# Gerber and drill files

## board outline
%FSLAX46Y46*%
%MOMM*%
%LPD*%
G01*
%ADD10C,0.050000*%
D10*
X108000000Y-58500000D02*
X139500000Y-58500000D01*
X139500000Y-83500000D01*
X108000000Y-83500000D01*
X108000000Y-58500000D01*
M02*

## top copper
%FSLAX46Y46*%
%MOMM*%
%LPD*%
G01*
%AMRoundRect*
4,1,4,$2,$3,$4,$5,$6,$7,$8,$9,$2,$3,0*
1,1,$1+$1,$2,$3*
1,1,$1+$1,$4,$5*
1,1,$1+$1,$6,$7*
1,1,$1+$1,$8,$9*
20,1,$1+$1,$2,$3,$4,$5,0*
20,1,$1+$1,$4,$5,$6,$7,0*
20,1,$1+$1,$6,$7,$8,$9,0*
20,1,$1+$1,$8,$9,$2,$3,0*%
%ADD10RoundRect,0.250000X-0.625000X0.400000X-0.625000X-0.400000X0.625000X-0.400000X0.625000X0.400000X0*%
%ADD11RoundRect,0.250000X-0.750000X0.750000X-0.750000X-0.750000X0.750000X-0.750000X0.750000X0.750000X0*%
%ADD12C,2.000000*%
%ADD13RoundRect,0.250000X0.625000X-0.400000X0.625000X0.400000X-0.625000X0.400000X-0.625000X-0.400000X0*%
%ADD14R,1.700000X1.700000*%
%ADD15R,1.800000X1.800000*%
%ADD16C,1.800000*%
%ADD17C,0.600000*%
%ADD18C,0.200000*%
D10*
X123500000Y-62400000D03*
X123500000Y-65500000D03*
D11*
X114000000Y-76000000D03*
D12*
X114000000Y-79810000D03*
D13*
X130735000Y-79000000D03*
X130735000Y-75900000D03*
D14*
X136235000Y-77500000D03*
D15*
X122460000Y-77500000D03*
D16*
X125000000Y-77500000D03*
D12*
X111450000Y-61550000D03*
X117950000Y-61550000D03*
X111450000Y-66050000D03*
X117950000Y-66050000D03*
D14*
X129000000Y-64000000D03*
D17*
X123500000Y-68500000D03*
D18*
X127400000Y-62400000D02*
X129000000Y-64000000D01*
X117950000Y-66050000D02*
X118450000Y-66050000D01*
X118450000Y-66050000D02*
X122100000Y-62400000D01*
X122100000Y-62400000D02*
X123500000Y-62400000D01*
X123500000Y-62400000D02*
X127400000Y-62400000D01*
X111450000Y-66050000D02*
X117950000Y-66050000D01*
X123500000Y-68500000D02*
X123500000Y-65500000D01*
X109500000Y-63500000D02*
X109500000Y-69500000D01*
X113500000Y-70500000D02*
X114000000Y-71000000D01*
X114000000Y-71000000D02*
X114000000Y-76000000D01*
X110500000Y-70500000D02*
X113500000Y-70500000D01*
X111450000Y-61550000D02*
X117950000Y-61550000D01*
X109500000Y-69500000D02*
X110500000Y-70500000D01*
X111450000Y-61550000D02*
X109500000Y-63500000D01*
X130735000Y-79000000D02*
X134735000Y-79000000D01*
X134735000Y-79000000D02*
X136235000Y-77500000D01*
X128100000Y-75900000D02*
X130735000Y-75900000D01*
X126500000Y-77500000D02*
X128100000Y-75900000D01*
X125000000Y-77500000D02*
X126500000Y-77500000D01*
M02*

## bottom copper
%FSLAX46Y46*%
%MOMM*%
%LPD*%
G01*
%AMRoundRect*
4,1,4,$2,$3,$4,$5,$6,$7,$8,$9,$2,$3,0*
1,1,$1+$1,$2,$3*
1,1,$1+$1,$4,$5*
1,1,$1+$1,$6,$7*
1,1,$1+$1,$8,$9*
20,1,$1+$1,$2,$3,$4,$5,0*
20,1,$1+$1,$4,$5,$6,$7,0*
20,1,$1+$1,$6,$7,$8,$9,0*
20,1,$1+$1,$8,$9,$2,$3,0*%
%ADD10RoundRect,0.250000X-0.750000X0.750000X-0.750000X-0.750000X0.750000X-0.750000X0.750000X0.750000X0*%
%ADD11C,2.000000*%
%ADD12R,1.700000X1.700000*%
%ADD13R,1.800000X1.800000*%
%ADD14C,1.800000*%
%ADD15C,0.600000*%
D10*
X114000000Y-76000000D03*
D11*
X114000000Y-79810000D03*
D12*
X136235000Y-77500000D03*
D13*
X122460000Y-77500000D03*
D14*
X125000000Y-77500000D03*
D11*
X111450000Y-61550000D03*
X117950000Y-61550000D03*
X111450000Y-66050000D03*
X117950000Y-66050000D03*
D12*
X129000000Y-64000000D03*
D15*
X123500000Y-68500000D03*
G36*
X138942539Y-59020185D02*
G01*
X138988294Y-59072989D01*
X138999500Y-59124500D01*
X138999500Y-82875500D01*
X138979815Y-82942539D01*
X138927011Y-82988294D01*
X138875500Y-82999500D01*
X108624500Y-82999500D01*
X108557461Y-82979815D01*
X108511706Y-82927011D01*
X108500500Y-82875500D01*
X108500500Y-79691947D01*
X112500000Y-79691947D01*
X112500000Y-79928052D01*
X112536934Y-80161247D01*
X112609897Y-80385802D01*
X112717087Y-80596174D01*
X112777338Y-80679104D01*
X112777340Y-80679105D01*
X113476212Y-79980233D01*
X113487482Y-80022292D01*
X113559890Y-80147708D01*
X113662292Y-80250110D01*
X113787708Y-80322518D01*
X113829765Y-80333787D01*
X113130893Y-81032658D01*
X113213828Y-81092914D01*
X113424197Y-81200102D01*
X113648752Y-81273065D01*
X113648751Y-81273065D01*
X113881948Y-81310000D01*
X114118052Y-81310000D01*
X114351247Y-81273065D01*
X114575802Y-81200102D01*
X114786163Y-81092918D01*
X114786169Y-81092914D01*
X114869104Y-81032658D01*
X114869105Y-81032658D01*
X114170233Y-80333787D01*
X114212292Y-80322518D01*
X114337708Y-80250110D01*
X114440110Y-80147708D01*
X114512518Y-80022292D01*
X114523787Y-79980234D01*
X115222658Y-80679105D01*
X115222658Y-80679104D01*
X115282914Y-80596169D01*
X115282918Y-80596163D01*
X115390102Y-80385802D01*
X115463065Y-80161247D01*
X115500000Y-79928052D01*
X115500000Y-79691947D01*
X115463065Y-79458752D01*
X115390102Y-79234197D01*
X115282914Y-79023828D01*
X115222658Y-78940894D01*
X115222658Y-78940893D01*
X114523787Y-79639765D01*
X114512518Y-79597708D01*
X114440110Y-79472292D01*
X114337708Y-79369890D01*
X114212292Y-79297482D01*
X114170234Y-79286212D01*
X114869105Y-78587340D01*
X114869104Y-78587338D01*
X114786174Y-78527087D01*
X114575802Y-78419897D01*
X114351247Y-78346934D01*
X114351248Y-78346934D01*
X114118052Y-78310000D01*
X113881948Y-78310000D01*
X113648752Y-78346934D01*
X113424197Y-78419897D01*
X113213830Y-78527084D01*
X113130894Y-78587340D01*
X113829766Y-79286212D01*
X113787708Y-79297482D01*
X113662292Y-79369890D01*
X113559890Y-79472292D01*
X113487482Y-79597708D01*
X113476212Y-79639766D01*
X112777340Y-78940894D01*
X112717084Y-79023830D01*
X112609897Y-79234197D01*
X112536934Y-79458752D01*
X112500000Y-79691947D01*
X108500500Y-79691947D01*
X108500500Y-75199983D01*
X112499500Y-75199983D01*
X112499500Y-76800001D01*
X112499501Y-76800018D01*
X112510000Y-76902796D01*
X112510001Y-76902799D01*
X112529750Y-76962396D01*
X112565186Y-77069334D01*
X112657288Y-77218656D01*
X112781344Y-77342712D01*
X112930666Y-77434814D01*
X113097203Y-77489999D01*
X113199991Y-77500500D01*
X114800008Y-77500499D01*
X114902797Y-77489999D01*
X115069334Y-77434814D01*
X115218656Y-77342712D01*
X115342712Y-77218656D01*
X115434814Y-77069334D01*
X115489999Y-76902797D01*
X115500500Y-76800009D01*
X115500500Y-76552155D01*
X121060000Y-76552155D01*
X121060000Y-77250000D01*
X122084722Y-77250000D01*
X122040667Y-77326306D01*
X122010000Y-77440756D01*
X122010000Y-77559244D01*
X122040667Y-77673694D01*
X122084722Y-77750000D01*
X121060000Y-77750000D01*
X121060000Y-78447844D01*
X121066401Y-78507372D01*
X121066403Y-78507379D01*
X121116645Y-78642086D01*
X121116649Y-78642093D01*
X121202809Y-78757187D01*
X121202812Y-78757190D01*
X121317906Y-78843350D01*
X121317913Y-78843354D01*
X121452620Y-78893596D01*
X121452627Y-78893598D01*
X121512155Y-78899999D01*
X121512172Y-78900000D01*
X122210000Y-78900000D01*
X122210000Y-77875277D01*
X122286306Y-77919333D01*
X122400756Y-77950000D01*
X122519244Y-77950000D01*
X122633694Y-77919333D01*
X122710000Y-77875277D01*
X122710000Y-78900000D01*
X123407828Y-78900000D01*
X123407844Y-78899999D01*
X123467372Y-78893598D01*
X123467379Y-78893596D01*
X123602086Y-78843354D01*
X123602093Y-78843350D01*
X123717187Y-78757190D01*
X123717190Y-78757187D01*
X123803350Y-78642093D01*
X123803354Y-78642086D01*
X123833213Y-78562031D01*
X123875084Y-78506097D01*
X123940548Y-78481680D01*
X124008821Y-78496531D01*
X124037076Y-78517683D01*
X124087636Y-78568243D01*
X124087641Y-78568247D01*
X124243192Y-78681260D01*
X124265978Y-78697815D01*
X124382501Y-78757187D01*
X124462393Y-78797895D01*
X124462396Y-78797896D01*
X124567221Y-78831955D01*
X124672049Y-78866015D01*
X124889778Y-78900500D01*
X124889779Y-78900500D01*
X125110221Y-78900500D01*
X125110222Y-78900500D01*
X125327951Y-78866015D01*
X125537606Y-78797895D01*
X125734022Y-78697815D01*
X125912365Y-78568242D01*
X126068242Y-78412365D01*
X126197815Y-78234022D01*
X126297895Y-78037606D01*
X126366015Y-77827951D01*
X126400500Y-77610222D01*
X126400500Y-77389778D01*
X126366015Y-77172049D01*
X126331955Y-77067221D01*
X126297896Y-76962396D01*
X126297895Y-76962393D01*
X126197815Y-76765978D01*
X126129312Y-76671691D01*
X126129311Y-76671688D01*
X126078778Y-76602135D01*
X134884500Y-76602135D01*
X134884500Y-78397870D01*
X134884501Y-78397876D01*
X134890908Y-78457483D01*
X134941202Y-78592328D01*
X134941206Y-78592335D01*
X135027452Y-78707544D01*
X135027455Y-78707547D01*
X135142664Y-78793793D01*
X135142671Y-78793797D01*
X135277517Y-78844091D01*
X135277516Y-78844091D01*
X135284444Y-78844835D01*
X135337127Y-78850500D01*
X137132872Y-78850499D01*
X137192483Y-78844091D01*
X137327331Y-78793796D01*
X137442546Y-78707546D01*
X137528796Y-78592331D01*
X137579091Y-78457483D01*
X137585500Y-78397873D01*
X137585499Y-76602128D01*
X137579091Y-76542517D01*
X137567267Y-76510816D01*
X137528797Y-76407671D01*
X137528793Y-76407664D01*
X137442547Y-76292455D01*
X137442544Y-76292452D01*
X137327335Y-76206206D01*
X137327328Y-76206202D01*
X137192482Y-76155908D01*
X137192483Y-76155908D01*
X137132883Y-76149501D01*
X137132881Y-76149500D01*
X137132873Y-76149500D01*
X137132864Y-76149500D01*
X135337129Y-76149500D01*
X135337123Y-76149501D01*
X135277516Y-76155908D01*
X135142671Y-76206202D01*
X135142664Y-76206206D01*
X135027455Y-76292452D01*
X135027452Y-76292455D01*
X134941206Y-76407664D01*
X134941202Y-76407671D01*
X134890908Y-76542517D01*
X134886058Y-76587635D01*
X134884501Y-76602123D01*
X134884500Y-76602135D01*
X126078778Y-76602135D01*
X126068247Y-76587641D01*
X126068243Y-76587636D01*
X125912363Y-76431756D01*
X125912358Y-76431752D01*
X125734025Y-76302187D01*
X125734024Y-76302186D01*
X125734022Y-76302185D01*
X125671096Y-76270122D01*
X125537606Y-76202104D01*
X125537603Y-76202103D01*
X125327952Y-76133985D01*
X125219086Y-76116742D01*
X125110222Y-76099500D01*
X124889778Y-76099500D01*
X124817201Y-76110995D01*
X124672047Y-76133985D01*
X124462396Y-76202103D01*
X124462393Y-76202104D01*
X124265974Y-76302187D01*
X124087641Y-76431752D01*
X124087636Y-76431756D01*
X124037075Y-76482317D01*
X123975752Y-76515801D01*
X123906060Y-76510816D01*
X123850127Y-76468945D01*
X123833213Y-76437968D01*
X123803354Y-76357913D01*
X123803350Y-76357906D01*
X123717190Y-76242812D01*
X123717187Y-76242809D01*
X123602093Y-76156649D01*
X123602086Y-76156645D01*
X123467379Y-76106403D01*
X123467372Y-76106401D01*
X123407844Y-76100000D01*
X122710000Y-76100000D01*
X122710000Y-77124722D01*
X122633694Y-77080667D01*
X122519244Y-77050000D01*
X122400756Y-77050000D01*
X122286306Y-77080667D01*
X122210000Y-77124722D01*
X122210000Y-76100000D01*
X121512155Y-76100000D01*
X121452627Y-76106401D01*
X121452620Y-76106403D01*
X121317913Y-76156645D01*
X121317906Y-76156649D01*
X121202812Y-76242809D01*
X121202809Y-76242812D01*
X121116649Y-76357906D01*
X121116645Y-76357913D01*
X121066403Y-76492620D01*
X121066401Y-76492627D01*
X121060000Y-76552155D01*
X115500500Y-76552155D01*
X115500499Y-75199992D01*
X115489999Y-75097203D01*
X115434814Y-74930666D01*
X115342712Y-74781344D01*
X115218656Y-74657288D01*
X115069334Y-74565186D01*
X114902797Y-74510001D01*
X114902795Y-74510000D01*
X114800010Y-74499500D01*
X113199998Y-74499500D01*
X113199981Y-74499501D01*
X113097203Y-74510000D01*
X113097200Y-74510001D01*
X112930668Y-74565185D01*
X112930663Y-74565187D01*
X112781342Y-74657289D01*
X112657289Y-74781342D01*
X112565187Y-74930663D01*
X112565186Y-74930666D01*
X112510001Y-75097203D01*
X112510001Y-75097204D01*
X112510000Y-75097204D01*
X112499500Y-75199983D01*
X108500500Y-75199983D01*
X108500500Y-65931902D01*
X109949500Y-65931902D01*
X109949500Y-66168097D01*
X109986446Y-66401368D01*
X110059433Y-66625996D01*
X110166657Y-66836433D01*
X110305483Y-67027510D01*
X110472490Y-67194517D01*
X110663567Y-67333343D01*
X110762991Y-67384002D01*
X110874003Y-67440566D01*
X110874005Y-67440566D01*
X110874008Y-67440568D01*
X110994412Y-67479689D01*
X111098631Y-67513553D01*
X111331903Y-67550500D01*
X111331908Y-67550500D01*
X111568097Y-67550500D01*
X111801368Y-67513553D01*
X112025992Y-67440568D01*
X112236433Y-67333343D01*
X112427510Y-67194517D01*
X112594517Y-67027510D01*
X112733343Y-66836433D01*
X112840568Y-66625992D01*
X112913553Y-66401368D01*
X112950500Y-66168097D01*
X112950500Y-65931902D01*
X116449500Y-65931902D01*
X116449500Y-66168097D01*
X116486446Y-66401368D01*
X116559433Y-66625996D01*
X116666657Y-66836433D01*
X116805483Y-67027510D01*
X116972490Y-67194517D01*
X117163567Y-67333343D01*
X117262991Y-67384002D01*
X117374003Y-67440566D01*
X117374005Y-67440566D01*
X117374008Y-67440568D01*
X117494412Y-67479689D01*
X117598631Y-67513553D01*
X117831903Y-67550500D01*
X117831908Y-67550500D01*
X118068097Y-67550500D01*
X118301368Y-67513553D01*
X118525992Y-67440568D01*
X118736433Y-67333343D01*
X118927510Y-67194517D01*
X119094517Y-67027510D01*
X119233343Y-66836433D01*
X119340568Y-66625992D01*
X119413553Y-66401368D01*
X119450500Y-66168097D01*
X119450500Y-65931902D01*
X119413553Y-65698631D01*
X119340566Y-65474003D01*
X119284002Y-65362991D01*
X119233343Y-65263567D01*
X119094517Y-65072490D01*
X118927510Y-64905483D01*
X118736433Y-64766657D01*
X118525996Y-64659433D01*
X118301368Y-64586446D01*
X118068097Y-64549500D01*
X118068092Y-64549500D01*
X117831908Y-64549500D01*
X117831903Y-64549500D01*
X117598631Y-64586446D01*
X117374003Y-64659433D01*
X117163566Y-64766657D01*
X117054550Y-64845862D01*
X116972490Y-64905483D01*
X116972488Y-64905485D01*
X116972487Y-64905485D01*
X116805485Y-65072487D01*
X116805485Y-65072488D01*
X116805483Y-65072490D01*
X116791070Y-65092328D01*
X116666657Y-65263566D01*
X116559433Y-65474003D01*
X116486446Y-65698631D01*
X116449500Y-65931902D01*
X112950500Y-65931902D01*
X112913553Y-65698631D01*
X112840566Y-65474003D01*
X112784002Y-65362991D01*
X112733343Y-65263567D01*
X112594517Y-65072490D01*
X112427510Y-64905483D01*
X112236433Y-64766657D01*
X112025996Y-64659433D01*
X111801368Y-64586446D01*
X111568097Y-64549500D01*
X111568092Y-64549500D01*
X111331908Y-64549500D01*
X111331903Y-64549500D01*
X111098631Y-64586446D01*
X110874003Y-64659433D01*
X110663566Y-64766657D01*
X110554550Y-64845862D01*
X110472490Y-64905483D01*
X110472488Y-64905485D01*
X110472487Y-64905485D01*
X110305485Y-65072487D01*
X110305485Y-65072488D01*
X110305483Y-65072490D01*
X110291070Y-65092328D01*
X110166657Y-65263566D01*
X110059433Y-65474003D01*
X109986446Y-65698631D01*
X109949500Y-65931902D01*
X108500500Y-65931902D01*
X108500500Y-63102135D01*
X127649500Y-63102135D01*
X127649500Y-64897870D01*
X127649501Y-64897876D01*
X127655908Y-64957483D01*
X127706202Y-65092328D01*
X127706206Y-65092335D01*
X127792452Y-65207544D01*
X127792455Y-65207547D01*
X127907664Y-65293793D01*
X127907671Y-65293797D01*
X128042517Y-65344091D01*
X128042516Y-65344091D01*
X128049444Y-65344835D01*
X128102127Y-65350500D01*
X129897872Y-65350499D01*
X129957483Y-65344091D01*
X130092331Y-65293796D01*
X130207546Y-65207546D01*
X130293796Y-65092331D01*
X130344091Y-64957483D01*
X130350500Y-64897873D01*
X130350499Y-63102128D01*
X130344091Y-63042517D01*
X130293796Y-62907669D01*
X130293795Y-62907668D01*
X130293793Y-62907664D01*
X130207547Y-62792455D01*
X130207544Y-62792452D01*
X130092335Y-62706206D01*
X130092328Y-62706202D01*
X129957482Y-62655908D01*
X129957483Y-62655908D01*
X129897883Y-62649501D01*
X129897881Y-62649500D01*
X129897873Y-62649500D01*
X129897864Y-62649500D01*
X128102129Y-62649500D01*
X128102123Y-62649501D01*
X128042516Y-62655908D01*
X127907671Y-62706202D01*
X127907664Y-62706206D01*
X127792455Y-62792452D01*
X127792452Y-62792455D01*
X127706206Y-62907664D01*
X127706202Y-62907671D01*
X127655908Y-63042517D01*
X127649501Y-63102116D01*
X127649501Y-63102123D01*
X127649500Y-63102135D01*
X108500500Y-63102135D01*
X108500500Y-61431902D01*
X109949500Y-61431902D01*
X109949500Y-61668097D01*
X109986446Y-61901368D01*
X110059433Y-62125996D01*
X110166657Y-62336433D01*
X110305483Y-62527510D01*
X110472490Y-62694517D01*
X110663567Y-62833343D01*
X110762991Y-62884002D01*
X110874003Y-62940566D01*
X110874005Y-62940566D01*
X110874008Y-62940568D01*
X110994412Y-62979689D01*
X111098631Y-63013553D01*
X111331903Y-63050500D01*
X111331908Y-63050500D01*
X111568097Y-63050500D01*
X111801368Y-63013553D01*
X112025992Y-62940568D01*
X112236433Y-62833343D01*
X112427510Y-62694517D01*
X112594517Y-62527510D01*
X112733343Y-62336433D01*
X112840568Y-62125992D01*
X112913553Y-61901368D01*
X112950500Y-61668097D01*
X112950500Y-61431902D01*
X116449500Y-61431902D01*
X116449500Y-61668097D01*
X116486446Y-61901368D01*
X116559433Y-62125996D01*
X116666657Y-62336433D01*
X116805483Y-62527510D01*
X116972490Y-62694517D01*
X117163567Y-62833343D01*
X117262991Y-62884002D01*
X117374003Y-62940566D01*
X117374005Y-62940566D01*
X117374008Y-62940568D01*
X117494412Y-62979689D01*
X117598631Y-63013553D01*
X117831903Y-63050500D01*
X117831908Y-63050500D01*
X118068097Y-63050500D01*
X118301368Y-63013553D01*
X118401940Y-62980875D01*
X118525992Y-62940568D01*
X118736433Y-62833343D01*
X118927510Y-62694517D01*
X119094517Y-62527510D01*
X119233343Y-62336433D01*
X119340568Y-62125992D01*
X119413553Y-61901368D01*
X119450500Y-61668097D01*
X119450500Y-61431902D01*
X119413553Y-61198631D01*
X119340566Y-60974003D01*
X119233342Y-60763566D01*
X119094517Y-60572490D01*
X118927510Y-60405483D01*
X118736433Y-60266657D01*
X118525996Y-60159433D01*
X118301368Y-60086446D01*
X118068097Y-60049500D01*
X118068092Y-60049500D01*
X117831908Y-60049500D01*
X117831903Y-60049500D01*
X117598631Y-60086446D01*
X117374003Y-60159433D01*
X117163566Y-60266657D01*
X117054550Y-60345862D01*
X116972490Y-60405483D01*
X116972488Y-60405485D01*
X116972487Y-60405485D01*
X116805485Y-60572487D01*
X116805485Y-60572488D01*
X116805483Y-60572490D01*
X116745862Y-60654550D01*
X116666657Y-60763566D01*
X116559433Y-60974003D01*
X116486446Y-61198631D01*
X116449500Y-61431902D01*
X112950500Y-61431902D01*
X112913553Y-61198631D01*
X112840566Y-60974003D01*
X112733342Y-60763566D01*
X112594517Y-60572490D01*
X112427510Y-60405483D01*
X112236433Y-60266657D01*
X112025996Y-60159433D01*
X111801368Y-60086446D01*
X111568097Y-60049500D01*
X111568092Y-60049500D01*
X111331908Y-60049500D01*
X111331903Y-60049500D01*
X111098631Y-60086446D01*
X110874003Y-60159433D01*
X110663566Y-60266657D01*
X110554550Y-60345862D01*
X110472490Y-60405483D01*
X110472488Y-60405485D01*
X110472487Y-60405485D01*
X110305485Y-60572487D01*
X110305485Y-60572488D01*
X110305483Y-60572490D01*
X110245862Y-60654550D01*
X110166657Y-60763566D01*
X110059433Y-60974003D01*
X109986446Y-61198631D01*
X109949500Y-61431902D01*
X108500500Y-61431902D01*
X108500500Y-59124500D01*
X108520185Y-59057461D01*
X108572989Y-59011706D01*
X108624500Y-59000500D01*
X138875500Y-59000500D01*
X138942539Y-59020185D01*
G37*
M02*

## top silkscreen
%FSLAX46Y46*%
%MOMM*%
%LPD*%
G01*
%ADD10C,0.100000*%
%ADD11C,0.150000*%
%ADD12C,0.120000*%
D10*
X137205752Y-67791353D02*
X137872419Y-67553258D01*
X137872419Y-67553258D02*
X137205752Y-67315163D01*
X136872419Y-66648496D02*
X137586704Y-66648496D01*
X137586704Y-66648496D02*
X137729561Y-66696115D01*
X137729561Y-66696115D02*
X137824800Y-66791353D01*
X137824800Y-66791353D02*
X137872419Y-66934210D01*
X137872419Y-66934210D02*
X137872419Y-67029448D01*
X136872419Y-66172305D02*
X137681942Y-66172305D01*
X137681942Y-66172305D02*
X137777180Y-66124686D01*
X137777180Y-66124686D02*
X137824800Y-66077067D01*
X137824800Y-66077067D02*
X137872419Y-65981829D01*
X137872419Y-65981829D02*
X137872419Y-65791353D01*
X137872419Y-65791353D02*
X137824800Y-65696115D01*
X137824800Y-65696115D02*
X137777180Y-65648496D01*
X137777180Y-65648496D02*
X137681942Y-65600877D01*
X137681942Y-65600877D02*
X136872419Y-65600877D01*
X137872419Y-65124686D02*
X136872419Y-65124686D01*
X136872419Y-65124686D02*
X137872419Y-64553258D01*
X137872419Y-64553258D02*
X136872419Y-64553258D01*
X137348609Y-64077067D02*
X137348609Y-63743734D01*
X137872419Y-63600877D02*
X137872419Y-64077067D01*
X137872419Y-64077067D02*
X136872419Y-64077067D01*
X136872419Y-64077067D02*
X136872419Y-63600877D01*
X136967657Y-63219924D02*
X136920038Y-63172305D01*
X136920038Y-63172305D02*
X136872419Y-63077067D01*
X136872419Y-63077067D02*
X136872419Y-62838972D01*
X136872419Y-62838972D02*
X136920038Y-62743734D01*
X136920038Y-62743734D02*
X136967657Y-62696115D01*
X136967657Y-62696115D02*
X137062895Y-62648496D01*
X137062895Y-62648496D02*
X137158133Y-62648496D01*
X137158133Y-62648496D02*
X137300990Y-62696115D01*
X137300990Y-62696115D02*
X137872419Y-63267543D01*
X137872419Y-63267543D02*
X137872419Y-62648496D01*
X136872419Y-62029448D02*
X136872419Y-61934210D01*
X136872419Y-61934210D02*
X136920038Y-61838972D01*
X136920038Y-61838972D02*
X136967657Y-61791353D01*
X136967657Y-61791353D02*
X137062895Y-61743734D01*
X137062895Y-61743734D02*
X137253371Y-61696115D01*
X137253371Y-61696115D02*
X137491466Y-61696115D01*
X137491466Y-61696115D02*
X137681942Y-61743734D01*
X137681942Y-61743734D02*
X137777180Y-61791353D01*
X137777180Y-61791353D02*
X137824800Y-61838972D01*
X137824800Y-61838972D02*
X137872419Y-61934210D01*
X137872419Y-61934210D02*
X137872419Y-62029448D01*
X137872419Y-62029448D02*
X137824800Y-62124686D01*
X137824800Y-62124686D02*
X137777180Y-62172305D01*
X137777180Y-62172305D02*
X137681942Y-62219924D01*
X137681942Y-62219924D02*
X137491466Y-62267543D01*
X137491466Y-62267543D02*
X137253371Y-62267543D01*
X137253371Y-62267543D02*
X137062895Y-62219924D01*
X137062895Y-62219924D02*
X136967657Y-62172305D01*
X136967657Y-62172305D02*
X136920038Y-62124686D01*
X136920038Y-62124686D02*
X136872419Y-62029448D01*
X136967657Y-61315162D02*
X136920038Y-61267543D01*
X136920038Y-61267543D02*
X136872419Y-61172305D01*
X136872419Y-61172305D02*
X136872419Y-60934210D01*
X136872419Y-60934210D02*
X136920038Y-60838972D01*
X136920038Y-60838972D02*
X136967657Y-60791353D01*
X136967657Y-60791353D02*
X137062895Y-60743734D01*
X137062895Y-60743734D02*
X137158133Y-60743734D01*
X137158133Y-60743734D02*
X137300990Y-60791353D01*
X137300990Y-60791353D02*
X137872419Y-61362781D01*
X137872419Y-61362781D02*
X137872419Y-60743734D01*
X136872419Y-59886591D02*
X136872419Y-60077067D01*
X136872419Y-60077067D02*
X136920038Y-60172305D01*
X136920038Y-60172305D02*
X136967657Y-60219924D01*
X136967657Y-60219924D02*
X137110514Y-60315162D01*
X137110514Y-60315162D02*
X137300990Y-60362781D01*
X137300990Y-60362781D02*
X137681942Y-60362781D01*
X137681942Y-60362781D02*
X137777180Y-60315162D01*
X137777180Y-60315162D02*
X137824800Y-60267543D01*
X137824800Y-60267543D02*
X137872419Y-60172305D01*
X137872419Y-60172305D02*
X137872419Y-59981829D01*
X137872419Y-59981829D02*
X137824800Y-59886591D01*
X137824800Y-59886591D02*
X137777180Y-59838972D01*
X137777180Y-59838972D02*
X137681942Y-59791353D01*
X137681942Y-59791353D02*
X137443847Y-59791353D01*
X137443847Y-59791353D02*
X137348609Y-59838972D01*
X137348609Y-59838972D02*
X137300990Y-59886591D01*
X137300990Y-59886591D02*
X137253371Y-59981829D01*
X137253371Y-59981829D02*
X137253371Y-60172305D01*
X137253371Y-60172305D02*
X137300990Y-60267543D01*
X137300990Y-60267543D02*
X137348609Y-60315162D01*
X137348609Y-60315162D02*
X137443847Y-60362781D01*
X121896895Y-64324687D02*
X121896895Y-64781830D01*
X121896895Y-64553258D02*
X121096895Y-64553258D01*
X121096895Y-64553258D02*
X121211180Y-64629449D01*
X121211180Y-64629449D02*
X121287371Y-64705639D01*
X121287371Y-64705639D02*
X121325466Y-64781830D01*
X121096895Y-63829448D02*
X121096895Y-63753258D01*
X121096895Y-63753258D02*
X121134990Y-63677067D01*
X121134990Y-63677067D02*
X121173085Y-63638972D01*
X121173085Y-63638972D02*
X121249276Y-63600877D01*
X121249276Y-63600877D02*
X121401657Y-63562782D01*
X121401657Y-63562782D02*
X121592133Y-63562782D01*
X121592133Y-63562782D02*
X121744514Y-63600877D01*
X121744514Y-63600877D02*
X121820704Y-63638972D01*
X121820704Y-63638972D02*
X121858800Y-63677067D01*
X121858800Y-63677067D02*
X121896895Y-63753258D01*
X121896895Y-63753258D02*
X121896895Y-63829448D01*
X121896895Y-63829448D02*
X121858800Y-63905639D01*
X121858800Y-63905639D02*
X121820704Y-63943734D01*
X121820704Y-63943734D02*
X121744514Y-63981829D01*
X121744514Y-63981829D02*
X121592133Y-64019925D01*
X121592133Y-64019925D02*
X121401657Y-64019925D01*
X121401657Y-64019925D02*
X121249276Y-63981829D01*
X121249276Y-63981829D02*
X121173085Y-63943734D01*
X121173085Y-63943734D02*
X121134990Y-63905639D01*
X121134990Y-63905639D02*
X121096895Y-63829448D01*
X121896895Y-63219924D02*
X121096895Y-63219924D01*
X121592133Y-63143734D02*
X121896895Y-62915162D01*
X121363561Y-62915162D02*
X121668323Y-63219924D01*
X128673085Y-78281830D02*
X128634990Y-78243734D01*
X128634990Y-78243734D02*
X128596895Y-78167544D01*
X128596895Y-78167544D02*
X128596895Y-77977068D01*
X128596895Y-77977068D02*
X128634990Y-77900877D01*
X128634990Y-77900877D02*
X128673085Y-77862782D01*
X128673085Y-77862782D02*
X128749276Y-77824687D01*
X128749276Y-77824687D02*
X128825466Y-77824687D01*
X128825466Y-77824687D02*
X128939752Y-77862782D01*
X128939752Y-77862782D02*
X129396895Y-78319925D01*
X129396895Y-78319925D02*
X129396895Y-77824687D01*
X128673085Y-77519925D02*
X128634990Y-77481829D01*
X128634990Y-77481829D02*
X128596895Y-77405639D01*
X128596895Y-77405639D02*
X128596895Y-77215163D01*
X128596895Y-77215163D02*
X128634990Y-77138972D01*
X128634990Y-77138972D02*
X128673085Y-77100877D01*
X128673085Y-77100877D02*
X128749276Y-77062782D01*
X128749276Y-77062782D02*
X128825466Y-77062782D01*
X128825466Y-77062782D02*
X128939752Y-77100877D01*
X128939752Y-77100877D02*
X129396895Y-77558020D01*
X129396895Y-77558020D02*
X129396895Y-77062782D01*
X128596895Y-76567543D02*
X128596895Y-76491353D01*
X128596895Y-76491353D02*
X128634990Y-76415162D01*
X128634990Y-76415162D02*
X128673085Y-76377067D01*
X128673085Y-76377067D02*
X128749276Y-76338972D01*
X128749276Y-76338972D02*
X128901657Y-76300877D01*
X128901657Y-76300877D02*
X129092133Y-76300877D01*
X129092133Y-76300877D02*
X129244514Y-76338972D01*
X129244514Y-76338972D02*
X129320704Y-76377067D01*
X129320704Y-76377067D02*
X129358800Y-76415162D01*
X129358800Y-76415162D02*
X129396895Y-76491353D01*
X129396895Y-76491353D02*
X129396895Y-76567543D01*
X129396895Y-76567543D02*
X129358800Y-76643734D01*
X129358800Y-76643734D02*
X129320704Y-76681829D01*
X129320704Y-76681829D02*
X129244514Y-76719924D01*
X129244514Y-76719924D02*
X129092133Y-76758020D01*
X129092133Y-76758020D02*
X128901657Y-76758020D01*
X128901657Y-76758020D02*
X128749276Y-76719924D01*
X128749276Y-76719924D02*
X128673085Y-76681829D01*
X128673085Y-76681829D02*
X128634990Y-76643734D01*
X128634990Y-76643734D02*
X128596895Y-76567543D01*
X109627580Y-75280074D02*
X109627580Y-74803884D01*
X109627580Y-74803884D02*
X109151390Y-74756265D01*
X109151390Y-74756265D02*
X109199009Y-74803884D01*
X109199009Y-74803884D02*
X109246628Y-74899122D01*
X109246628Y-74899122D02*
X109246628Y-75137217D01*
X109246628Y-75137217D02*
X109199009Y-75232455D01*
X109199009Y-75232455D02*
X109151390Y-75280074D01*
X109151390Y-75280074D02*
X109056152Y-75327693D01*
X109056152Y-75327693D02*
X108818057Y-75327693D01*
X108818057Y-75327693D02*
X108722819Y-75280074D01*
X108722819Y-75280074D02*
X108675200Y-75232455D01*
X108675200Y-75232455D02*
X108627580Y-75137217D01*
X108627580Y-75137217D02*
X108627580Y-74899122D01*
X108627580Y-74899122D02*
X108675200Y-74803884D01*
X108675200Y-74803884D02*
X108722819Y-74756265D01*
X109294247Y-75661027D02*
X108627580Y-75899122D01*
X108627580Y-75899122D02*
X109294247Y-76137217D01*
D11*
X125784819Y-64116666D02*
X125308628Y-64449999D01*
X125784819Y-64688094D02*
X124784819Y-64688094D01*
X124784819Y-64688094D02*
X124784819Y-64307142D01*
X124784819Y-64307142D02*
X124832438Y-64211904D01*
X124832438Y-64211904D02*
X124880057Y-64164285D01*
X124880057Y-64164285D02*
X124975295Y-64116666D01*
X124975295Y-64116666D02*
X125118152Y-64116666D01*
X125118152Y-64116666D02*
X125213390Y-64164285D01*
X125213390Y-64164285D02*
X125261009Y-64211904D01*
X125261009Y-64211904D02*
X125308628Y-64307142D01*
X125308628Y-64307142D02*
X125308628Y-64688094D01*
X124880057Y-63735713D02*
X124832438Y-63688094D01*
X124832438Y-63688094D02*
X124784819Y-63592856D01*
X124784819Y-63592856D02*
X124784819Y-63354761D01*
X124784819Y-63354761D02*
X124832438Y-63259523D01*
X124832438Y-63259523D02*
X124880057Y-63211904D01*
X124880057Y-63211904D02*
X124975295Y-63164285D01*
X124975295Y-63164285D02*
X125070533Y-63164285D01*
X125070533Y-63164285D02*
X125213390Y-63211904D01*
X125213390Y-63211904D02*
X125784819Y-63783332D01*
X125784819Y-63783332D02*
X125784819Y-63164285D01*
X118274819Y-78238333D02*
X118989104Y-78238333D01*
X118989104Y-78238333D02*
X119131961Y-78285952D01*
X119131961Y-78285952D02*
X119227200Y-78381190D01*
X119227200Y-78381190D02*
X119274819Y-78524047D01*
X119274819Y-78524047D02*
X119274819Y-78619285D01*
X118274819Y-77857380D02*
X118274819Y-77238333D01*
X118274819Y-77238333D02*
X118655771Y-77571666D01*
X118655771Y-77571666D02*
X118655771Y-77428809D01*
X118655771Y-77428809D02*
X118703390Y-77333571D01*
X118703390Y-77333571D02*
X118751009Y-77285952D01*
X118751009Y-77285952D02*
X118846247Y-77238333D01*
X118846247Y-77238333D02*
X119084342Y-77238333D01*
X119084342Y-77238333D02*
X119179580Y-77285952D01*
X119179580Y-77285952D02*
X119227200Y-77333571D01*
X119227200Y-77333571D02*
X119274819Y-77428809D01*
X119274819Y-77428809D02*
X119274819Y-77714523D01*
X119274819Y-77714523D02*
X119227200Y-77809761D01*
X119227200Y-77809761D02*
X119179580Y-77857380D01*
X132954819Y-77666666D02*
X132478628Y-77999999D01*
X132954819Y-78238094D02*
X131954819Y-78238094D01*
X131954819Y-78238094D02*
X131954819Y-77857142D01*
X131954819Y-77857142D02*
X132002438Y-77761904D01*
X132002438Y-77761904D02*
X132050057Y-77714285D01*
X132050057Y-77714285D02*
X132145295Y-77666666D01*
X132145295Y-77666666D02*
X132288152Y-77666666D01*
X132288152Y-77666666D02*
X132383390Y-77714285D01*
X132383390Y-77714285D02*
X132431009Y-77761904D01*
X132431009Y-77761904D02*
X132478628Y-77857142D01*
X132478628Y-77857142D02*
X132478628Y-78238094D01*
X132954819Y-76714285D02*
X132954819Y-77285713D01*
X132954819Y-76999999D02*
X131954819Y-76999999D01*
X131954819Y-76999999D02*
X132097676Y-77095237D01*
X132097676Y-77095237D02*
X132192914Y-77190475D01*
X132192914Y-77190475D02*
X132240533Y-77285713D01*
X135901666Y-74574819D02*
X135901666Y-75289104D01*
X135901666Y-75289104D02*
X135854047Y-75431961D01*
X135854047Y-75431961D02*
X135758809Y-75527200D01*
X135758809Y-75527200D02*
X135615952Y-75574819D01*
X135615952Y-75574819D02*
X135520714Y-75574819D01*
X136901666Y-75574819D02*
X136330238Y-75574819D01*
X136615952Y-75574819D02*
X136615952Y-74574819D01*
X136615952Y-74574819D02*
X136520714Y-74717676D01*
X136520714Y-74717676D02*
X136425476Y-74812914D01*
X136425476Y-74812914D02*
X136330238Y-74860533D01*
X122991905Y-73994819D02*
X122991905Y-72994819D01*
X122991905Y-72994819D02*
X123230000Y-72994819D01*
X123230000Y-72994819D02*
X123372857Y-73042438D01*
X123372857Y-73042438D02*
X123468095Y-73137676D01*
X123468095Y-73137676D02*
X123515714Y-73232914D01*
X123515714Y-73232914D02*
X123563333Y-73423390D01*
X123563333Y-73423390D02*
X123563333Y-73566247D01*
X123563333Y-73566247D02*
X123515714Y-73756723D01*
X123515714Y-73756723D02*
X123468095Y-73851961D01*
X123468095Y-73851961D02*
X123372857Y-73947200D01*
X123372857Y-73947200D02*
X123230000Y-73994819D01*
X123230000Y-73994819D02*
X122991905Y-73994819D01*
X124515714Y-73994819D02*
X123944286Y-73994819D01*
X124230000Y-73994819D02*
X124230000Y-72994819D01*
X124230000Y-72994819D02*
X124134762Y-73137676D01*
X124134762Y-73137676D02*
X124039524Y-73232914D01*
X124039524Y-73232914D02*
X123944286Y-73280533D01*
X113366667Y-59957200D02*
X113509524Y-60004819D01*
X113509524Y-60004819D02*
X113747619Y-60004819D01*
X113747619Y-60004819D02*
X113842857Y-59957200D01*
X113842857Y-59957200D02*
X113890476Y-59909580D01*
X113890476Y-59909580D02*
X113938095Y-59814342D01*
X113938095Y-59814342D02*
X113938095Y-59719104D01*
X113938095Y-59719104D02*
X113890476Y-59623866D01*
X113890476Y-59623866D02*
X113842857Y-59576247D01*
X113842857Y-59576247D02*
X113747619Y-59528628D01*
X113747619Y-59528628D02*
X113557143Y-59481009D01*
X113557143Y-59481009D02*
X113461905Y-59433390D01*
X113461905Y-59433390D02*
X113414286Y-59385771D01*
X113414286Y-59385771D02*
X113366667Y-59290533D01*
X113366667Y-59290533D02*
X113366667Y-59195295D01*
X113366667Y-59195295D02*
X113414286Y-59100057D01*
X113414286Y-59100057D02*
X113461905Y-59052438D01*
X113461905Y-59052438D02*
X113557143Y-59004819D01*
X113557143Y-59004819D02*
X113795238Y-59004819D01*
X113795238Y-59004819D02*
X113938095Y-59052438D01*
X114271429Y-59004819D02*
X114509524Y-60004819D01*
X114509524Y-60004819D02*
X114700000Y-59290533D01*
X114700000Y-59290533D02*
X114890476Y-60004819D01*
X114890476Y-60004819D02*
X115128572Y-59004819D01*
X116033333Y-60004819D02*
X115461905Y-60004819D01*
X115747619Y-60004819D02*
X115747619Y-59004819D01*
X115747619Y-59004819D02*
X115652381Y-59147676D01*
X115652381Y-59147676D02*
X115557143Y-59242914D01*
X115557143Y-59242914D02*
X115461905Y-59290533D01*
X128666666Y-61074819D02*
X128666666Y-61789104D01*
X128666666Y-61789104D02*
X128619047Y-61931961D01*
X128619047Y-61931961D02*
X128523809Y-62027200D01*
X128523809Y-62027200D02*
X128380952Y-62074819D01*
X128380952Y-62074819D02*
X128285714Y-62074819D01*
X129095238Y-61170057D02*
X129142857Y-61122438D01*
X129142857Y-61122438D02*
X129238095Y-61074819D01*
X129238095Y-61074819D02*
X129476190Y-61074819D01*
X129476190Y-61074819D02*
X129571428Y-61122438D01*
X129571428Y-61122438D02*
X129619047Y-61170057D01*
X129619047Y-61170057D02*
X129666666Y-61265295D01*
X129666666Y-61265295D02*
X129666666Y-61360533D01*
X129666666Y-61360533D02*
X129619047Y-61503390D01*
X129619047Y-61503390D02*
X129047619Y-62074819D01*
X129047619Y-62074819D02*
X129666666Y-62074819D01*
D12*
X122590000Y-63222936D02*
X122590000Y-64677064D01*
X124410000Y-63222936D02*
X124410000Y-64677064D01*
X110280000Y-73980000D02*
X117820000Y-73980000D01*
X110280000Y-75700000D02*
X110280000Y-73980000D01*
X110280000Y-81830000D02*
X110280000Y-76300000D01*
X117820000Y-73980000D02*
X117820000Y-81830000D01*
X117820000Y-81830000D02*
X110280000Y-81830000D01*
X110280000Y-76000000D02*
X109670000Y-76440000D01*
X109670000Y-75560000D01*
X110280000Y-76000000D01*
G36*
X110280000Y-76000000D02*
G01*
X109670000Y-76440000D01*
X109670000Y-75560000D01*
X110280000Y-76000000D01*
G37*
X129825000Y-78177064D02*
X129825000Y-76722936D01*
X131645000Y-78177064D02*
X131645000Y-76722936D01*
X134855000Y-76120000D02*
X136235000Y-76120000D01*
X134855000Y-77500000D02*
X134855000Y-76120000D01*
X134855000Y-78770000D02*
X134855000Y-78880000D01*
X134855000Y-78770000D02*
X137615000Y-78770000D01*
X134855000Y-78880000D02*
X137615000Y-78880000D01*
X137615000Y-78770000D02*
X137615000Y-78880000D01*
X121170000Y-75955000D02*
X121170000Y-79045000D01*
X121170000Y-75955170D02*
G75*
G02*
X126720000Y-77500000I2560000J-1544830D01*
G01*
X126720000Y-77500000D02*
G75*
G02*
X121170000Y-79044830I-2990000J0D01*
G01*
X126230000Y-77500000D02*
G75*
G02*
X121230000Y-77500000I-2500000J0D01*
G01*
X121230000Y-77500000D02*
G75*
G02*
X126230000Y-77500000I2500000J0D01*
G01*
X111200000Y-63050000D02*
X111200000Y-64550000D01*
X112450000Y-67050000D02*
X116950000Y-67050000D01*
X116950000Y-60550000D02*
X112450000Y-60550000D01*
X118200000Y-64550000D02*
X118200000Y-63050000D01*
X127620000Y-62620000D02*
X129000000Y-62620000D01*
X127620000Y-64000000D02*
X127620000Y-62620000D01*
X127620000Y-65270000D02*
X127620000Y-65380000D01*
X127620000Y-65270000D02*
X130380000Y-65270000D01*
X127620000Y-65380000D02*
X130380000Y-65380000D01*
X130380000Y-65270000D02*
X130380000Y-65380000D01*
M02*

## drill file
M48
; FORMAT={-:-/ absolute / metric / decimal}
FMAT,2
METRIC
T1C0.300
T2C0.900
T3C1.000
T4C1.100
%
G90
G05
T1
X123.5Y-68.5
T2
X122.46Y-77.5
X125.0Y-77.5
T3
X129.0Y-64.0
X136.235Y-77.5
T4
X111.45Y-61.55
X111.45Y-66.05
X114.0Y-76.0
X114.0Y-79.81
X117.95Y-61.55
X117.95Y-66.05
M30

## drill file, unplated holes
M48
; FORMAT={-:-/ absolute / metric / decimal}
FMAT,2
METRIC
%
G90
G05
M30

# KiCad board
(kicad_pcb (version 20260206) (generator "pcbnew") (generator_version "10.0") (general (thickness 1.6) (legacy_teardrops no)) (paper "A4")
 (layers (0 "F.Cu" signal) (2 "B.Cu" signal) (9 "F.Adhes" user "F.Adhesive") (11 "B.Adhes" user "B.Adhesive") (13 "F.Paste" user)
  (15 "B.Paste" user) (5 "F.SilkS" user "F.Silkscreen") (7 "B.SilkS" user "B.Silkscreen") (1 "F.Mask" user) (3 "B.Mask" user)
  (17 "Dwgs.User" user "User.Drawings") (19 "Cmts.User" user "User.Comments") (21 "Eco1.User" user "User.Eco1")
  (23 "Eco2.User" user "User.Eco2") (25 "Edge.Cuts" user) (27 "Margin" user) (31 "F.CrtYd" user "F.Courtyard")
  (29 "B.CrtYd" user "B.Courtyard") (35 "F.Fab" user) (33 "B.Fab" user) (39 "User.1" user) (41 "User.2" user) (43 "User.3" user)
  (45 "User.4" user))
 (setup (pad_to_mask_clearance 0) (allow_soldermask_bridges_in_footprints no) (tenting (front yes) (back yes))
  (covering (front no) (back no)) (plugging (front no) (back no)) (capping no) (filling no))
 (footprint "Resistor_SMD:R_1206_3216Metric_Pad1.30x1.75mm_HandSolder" (layer "F.Cu") (at 123.5 63.95 -90)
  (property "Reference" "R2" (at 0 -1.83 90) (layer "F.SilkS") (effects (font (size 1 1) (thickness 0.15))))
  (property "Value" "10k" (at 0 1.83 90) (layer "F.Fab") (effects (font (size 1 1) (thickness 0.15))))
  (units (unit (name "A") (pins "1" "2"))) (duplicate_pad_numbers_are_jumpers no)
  (fp_line (start -0.727064 0.91) (end 0.727064 0.91) (stroke (width 0.12) (type solid)) (layer "F.SilkS"))
  (fp_line (start -0.727064 -0.91) (end 0.727064 -0.91) (stroke (width 0.12) (type solid)) (layer "F.SilkS"))
  (pad "1" smd roundrect (at -1.55 0 270) (size 1.3 1.75) (layers "F.Cu" "F.Mask" "F.Paste") (roundrect_rratio 0.192308)
   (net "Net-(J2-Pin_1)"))
  (pad "2" smd roundrect (at 1.55 0 270) (size 1.3 1.75) (layers "F.Cu" "F.Mask" "F.Paste") (roundrect_rratio 0.192308) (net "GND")))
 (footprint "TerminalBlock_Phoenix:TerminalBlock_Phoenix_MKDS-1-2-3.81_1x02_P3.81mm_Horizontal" (layer "F.Cu") (at 114 76 -90)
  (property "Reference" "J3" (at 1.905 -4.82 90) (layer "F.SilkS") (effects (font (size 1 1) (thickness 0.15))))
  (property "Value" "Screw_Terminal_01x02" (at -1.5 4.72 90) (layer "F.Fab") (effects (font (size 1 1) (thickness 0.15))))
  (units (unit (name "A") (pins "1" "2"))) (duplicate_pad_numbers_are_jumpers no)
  (fp_line (start -2.02 3.72) (end -2.02 -3.82) (stroke (width 0.12) (type solid)) (layer "F.SilkS"))
  (fp_line (start -0.3 3.72) (end -2.02 3.72) (stroke (width 0.12) (type solid)) (layer "F.SilkS"))
  (fp_line (start 5.83 3.72) (end 0.3 3.72) (stroke (width 0.12) (type solid)) (layer "F.SilkS"))
  (fp_line (start -2.02 -3.82) (end 5.83 -3.82) (stroke (width 0.12) (type solid)) (layer "F.SilkS"))
  (fp_line (start 5.83 -3.82) (end 5.83 3.72) (stroke (width 0.12) (type solid)) (layer "F.SilkS"))
  (fp_poly (pts (xy 0 3.72) (xy 0.44 4.33) (xy -0.44 4.33)) (stroke (width 0.12) (type solid)) (fill yes) (layer "F.SilkS"))
  (pad "1" thru_hole roundrect (at 0 0 270) (size 2 2) (drill 1.1) (layers "*.Cu" "*.Mask") (remove_unused_layers no)
   (roundrect_rratio 0.125) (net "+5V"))
  (pad "2" thru_hole circle (at 3.81 0 270) (size 2 2) (drill 1.1) (layers "*.Cu" "*.Mask") (remove_unused_layers no) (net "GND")))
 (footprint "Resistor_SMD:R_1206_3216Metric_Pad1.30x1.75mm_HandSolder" (layer "F.Cu") (at 130.735 77.45 90)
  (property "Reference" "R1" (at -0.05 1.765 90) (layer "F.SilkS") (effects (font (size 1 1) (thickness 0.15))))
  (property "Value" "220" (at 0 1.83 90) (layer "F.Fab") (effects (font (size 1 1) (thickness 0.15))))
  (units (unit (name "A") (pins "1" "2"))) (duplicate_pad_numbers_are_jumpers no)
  (fp_line (start -0.727064 -0.91) (end 0.727064 -0.91) (stroke (width 0.12) (type solid)) (layer "F.SilkS"))
  (fp_line (start -0.727064 0.91) (end 0.727064 0.91) (stroke (width 0.12) (type solid)) (layer "F.SilkS"))
  (pad "1" smd roundrect (at -1.55 0 90) (size 1.3 1.75) (layers "F.Cu" "F.Mask" "F.Paste") (roundrect_rratio 0.192308)
   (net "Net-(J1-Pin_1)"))
  (pad "2" smd roundrect (at 1.55 0 90) (size 1.3 1.75) (layers "F.Cu" "F.Mask" "F.Paste") (roundrect_rratio 0.192308) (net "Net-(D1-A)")))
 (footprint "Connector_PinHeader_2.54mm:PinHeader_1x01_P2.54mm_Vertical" (layer "F.Cu") (at 136.235 77.5)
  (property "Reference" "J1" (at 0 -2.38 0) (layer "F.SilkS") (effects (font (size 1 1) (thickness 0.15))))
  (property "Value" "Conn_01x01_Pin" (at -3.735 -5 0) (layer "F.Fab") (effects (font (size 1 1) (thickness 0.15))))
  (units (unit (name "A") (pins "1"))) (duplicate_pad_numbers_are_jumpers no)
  (fp_line (start -1.38 -1.38) (end 0 -1.38) (stroke (width 0.12) (type solid)) (layer "F.SilkS"))
  (fp_line (start -1.38 0) (end -1.38 -1.38) (stroke (width 0.12) (type solid)) (layer "F.SilkS"))
  (fp_line (start -1.38 1.27) (end -1.38 1.38) (stroke (width 0.12) (type solid)) (layer "F.SilkS"))
  (fp_line (start -1.38 1.27) (end 1.38 1.27) (stroke (width 0.12) (type solid)) (layer "F.SilkS"))
  (fp_line (start -1.38 1.38) (end 1.38 1.38) (stroke (width 0.12) (type solid)) (layer "F.SilkS"))
  (fp_line (start 1.38 1.27) (end 1.38 1.38) (stroke (width 0.12) (type solid)) (layer "F.SilkS"))
  (pad "1" thru_hole rect (at 0 0) (size 1.7 1.7) (drill 1) (layers "*.Cu" "*.Mask") (remove_unused_layers no) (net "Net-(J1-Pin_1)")))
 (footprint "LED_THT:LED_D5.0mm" (layer "F.Cu") (at 122.46 77.5)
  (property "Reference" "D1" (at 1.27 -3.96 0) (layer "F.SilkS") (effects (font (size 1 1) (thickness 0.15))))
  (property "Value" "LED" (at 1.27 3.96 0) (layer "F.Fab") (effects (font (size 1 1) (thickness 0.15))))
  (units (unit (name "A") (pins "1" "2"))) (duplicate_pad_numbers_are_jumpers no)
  (fp_line (start -1.29 -1.545) (end -1.29 1.545) (stroke (width 0.12) (type solid)) (layer "F.SilkS"))
  (fp_arc (start -1.29 -1.54483) (mid 2.071779 -2.880495) (end 4.26 0) (stroke (width 0.12) (type solid)) (layer "F.SilkS"))
  (fp_arc (start 4.26 0) (mid 2.071779 2.880495) (end -1.29 1.54483) (stroke (width 0.12) (type solid)) (layer "F.SilkS"))
  (fp_circle (center 1.27 0) (end 3.77 0) (stroke (width 0.12) (type solid)) (fill no) (layer "F.SilkS"))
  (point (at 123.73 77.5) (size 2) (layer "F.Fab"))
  (pad "1" thru_hole rect (at 0 0) (size 1.8 1.8) (drill 0.9) (layers "*.Cu" "*.Mask") (remove_unused_layers no) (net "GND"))
  (pad "2" thru_hole circle (at 2.54 0) (size 1.8 1.8) (drill 0.9) (layers "*.Cu" "*.Mask") (remove_unused_layers no) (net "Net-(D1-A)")))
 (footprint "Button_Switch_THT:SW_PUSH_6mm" (layer "F.Cu") (at 111.45 61.55)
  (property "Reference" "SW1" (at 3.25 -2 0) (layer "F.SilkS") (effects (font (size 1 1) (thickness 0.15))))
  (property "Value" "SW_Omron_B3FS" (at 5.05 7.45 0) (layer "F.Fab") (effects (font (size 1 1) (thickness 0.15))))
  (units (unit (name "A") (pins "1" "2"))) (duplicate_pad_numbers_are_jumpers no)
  (fp_line (start -0.25 1.5) (end -0.25 3) (stroke (width 0.12) (type solid)) (layer "F.SilkS"))
  (fp_line (start 1 5.5) (end 5.5 5.5) (stroke (width 0.12) (type solid)) (layer "F.SilkS"))
  (fp_line (start 5.5 -1) (end 1 -1) (stroke (width 0.12) (type solid)) (layer "F.SilkS"))
  (fp_line (start 6.75 3) (end 6.75 1.5) (stroke (width 0.12) (type solid)) (layer "F.SilkS"))
  (pad "1" thru_hole circle (at 0 0 90) (size 2 2) (drill 1.1) (layers "*.Cu" "*.Mask") (remove_unused_layers no) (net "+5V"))
  (pad "1" thru_hole circle (at 6.5 0 90) (size 2 2) (drill 1.1) (layers "*.Cu" "*.Mask") (remove_unused_layers no) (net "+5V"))
  (pad "2" thru_hole circle (at 0 4.5 90) (size 2 2) (drill 1.1) (layers "*.Cu" "*.Mask") (remove_unused_layers no) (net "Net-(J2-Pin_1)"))
  (pad "2" thru_hole circle (at 6.5 4.5 90) (size 2 2) (drill 1.1) (layers "*.Cu" "*.Mask") (remove_unused_layers no) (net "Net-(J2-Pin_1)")))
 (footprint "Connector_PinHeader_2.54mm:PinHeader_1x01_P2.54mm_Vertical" (layer "F.Cu") (at 129 64)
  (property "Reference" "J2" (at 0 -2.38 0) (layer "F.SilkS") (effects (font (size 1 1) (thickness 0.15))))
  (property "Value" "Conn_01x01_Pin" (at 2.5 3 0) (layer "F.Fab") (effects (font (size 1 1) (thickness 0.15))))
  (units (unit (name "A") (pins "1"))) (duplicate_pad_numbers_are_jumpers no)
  (fp_line (start -1.38 -1.38) (end 0 -1.38) (stroke (width 0.12) (type solid)) (layer "F.SilkS"))
  (fp_line (start -1.38 0) (end -1.38 -1.38) (stroke (width 0.12) (type solid)) (layer "F.SilkS"))
  (fp_line (start -1.38 1.27) (end -1.38 1.38) (stroke (width 0.12) (type solid)) (layer "F.SilkS"))
  (fp_line (start -1.38 1.27) (end 1.38 1.27) (stroke (width 0.12) (type solid)) (layer "F.SilkS"))
  (fp_line (start -1.38 1.38) (end 1.38 1.38) (stroke (width 0.12) (type solid)) (layer "F.SilkS"))
  (fp_line (start 1.38 1.27) (end 1.38 1.38) (stroke (width 0.12) (type solid)) (layer "F.SilkS"))
  (pad "1" thru_hole rect (at 0 0) (size 1.7 1.7) (drill 1) (layers "*.Cu" "*.Mask") (remove_unused_layers no) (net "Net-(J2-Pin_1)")))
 (gr_rect (start 108 58.5) (end 139.5 83.5) (stroke (width 0.05) (type default)) (fill no) (layer "Edge.Cuts"))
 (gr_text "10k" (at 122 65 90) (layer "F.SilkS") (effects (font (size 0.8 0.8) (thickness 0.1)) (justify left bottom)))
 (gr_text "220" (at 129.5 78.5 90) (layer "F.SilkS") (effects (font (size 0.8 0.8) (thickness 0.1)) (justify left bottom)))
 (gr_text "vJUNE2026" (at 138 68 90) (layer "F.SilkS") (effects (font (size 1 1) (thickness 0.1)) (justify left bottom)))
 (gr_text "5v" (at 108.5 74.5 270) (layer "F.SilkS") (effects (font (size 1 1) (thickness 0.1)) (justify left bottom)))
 (segment (start 127.4 62.4) (end 129 64) (width 0.2) (layer "F.Cu") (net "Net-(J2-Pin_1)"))
 (segment (start 117.95 66.05) (end 118.45 66.05) (width 0.2) (layer "F.Cu") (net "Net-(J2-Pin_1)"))
 (segment (start 118.45 66.05) (end 122.1 62.4) (width 0.2) (layer "F.Cu") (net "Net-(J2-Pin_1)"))
 (segment (start 122.1 62.4) (end 123.5 62.4) (width 0.2) (layer "F.Cu") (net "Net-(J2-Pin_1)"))
 (segment (start 123.5 62.4) (end 127.4 62.4) (width 0.2) (layer "F.Cu") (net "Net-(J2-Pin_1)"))
 (segment (start 111.45 66.05) (end 117.95 66.05) (width 0.2) (layer "F.Cu") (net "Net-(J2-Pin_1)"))
 (segment (start 123.5 68.5) (end 123.5 65.5) (width 0.2) (layer "F.Cu") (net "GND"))
 (via (at 123.5 68.5) (size 0.6) (drill 0.3) (layers "F.Cu" "B.Cu") (free yes) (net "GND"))
 (segment (start 109.5 63.5) (end 109.5 69.5) (width 0.2) (layer "F.Cu") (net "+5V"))
 (segment (start 113.5 70.5) (end 114 71) (width 0.2) (layer "F.Cu") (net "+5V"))
 (segment (start 114 71) (end 114 76) (width 0.2) (layer "F.Cu") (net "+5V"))
 (segment (start 110.5 70.5) (end 113.5 70.5) (width 0.2) (layer "F.Cu") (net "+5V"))
 (segment (start 111.45 61.55) (end 117.95 61.55) (width 0.2) (layer "F.Cu") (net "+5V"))
 (segment (start 109.5 69.5) (end 110.5 70.5) (width 0.2) (layer "F.Cu") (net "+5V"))
 (segment (start 111.45 61.55) (end 109.5 63.5) (width 0.2) (layer "F.Cu") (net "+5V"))
 (segment (start 130.735 79) (end 134.735 79) (width 0.2) (layer "F.Cu") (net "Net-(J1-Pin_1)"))
 (segment (start 134.735 79) (end 136.235 77.5) (width 0.2) (layer "F.Cu") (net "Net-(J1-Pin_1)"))
 (segment (start 128.1 75.9) (end 130.735 75.9) (width 0.2) (layer "F.Cu") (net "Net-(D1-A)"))
 (segment (start 126.5 77.5) (end 128.1 75.9) (width 0.2) (layer "F.Cu") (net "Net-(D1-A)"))
 (segment (start 125 77.5) (end 126.5 77.5) (width 0.2) (layer "F.Cu") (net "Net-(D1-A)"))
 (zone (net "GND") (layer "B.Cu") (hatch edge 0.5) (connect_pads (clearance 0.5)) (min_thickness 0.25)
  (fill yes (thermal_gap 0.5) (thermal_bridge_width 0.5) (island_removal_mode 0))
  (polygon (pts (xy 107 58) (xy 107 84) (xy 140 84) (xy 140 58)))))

